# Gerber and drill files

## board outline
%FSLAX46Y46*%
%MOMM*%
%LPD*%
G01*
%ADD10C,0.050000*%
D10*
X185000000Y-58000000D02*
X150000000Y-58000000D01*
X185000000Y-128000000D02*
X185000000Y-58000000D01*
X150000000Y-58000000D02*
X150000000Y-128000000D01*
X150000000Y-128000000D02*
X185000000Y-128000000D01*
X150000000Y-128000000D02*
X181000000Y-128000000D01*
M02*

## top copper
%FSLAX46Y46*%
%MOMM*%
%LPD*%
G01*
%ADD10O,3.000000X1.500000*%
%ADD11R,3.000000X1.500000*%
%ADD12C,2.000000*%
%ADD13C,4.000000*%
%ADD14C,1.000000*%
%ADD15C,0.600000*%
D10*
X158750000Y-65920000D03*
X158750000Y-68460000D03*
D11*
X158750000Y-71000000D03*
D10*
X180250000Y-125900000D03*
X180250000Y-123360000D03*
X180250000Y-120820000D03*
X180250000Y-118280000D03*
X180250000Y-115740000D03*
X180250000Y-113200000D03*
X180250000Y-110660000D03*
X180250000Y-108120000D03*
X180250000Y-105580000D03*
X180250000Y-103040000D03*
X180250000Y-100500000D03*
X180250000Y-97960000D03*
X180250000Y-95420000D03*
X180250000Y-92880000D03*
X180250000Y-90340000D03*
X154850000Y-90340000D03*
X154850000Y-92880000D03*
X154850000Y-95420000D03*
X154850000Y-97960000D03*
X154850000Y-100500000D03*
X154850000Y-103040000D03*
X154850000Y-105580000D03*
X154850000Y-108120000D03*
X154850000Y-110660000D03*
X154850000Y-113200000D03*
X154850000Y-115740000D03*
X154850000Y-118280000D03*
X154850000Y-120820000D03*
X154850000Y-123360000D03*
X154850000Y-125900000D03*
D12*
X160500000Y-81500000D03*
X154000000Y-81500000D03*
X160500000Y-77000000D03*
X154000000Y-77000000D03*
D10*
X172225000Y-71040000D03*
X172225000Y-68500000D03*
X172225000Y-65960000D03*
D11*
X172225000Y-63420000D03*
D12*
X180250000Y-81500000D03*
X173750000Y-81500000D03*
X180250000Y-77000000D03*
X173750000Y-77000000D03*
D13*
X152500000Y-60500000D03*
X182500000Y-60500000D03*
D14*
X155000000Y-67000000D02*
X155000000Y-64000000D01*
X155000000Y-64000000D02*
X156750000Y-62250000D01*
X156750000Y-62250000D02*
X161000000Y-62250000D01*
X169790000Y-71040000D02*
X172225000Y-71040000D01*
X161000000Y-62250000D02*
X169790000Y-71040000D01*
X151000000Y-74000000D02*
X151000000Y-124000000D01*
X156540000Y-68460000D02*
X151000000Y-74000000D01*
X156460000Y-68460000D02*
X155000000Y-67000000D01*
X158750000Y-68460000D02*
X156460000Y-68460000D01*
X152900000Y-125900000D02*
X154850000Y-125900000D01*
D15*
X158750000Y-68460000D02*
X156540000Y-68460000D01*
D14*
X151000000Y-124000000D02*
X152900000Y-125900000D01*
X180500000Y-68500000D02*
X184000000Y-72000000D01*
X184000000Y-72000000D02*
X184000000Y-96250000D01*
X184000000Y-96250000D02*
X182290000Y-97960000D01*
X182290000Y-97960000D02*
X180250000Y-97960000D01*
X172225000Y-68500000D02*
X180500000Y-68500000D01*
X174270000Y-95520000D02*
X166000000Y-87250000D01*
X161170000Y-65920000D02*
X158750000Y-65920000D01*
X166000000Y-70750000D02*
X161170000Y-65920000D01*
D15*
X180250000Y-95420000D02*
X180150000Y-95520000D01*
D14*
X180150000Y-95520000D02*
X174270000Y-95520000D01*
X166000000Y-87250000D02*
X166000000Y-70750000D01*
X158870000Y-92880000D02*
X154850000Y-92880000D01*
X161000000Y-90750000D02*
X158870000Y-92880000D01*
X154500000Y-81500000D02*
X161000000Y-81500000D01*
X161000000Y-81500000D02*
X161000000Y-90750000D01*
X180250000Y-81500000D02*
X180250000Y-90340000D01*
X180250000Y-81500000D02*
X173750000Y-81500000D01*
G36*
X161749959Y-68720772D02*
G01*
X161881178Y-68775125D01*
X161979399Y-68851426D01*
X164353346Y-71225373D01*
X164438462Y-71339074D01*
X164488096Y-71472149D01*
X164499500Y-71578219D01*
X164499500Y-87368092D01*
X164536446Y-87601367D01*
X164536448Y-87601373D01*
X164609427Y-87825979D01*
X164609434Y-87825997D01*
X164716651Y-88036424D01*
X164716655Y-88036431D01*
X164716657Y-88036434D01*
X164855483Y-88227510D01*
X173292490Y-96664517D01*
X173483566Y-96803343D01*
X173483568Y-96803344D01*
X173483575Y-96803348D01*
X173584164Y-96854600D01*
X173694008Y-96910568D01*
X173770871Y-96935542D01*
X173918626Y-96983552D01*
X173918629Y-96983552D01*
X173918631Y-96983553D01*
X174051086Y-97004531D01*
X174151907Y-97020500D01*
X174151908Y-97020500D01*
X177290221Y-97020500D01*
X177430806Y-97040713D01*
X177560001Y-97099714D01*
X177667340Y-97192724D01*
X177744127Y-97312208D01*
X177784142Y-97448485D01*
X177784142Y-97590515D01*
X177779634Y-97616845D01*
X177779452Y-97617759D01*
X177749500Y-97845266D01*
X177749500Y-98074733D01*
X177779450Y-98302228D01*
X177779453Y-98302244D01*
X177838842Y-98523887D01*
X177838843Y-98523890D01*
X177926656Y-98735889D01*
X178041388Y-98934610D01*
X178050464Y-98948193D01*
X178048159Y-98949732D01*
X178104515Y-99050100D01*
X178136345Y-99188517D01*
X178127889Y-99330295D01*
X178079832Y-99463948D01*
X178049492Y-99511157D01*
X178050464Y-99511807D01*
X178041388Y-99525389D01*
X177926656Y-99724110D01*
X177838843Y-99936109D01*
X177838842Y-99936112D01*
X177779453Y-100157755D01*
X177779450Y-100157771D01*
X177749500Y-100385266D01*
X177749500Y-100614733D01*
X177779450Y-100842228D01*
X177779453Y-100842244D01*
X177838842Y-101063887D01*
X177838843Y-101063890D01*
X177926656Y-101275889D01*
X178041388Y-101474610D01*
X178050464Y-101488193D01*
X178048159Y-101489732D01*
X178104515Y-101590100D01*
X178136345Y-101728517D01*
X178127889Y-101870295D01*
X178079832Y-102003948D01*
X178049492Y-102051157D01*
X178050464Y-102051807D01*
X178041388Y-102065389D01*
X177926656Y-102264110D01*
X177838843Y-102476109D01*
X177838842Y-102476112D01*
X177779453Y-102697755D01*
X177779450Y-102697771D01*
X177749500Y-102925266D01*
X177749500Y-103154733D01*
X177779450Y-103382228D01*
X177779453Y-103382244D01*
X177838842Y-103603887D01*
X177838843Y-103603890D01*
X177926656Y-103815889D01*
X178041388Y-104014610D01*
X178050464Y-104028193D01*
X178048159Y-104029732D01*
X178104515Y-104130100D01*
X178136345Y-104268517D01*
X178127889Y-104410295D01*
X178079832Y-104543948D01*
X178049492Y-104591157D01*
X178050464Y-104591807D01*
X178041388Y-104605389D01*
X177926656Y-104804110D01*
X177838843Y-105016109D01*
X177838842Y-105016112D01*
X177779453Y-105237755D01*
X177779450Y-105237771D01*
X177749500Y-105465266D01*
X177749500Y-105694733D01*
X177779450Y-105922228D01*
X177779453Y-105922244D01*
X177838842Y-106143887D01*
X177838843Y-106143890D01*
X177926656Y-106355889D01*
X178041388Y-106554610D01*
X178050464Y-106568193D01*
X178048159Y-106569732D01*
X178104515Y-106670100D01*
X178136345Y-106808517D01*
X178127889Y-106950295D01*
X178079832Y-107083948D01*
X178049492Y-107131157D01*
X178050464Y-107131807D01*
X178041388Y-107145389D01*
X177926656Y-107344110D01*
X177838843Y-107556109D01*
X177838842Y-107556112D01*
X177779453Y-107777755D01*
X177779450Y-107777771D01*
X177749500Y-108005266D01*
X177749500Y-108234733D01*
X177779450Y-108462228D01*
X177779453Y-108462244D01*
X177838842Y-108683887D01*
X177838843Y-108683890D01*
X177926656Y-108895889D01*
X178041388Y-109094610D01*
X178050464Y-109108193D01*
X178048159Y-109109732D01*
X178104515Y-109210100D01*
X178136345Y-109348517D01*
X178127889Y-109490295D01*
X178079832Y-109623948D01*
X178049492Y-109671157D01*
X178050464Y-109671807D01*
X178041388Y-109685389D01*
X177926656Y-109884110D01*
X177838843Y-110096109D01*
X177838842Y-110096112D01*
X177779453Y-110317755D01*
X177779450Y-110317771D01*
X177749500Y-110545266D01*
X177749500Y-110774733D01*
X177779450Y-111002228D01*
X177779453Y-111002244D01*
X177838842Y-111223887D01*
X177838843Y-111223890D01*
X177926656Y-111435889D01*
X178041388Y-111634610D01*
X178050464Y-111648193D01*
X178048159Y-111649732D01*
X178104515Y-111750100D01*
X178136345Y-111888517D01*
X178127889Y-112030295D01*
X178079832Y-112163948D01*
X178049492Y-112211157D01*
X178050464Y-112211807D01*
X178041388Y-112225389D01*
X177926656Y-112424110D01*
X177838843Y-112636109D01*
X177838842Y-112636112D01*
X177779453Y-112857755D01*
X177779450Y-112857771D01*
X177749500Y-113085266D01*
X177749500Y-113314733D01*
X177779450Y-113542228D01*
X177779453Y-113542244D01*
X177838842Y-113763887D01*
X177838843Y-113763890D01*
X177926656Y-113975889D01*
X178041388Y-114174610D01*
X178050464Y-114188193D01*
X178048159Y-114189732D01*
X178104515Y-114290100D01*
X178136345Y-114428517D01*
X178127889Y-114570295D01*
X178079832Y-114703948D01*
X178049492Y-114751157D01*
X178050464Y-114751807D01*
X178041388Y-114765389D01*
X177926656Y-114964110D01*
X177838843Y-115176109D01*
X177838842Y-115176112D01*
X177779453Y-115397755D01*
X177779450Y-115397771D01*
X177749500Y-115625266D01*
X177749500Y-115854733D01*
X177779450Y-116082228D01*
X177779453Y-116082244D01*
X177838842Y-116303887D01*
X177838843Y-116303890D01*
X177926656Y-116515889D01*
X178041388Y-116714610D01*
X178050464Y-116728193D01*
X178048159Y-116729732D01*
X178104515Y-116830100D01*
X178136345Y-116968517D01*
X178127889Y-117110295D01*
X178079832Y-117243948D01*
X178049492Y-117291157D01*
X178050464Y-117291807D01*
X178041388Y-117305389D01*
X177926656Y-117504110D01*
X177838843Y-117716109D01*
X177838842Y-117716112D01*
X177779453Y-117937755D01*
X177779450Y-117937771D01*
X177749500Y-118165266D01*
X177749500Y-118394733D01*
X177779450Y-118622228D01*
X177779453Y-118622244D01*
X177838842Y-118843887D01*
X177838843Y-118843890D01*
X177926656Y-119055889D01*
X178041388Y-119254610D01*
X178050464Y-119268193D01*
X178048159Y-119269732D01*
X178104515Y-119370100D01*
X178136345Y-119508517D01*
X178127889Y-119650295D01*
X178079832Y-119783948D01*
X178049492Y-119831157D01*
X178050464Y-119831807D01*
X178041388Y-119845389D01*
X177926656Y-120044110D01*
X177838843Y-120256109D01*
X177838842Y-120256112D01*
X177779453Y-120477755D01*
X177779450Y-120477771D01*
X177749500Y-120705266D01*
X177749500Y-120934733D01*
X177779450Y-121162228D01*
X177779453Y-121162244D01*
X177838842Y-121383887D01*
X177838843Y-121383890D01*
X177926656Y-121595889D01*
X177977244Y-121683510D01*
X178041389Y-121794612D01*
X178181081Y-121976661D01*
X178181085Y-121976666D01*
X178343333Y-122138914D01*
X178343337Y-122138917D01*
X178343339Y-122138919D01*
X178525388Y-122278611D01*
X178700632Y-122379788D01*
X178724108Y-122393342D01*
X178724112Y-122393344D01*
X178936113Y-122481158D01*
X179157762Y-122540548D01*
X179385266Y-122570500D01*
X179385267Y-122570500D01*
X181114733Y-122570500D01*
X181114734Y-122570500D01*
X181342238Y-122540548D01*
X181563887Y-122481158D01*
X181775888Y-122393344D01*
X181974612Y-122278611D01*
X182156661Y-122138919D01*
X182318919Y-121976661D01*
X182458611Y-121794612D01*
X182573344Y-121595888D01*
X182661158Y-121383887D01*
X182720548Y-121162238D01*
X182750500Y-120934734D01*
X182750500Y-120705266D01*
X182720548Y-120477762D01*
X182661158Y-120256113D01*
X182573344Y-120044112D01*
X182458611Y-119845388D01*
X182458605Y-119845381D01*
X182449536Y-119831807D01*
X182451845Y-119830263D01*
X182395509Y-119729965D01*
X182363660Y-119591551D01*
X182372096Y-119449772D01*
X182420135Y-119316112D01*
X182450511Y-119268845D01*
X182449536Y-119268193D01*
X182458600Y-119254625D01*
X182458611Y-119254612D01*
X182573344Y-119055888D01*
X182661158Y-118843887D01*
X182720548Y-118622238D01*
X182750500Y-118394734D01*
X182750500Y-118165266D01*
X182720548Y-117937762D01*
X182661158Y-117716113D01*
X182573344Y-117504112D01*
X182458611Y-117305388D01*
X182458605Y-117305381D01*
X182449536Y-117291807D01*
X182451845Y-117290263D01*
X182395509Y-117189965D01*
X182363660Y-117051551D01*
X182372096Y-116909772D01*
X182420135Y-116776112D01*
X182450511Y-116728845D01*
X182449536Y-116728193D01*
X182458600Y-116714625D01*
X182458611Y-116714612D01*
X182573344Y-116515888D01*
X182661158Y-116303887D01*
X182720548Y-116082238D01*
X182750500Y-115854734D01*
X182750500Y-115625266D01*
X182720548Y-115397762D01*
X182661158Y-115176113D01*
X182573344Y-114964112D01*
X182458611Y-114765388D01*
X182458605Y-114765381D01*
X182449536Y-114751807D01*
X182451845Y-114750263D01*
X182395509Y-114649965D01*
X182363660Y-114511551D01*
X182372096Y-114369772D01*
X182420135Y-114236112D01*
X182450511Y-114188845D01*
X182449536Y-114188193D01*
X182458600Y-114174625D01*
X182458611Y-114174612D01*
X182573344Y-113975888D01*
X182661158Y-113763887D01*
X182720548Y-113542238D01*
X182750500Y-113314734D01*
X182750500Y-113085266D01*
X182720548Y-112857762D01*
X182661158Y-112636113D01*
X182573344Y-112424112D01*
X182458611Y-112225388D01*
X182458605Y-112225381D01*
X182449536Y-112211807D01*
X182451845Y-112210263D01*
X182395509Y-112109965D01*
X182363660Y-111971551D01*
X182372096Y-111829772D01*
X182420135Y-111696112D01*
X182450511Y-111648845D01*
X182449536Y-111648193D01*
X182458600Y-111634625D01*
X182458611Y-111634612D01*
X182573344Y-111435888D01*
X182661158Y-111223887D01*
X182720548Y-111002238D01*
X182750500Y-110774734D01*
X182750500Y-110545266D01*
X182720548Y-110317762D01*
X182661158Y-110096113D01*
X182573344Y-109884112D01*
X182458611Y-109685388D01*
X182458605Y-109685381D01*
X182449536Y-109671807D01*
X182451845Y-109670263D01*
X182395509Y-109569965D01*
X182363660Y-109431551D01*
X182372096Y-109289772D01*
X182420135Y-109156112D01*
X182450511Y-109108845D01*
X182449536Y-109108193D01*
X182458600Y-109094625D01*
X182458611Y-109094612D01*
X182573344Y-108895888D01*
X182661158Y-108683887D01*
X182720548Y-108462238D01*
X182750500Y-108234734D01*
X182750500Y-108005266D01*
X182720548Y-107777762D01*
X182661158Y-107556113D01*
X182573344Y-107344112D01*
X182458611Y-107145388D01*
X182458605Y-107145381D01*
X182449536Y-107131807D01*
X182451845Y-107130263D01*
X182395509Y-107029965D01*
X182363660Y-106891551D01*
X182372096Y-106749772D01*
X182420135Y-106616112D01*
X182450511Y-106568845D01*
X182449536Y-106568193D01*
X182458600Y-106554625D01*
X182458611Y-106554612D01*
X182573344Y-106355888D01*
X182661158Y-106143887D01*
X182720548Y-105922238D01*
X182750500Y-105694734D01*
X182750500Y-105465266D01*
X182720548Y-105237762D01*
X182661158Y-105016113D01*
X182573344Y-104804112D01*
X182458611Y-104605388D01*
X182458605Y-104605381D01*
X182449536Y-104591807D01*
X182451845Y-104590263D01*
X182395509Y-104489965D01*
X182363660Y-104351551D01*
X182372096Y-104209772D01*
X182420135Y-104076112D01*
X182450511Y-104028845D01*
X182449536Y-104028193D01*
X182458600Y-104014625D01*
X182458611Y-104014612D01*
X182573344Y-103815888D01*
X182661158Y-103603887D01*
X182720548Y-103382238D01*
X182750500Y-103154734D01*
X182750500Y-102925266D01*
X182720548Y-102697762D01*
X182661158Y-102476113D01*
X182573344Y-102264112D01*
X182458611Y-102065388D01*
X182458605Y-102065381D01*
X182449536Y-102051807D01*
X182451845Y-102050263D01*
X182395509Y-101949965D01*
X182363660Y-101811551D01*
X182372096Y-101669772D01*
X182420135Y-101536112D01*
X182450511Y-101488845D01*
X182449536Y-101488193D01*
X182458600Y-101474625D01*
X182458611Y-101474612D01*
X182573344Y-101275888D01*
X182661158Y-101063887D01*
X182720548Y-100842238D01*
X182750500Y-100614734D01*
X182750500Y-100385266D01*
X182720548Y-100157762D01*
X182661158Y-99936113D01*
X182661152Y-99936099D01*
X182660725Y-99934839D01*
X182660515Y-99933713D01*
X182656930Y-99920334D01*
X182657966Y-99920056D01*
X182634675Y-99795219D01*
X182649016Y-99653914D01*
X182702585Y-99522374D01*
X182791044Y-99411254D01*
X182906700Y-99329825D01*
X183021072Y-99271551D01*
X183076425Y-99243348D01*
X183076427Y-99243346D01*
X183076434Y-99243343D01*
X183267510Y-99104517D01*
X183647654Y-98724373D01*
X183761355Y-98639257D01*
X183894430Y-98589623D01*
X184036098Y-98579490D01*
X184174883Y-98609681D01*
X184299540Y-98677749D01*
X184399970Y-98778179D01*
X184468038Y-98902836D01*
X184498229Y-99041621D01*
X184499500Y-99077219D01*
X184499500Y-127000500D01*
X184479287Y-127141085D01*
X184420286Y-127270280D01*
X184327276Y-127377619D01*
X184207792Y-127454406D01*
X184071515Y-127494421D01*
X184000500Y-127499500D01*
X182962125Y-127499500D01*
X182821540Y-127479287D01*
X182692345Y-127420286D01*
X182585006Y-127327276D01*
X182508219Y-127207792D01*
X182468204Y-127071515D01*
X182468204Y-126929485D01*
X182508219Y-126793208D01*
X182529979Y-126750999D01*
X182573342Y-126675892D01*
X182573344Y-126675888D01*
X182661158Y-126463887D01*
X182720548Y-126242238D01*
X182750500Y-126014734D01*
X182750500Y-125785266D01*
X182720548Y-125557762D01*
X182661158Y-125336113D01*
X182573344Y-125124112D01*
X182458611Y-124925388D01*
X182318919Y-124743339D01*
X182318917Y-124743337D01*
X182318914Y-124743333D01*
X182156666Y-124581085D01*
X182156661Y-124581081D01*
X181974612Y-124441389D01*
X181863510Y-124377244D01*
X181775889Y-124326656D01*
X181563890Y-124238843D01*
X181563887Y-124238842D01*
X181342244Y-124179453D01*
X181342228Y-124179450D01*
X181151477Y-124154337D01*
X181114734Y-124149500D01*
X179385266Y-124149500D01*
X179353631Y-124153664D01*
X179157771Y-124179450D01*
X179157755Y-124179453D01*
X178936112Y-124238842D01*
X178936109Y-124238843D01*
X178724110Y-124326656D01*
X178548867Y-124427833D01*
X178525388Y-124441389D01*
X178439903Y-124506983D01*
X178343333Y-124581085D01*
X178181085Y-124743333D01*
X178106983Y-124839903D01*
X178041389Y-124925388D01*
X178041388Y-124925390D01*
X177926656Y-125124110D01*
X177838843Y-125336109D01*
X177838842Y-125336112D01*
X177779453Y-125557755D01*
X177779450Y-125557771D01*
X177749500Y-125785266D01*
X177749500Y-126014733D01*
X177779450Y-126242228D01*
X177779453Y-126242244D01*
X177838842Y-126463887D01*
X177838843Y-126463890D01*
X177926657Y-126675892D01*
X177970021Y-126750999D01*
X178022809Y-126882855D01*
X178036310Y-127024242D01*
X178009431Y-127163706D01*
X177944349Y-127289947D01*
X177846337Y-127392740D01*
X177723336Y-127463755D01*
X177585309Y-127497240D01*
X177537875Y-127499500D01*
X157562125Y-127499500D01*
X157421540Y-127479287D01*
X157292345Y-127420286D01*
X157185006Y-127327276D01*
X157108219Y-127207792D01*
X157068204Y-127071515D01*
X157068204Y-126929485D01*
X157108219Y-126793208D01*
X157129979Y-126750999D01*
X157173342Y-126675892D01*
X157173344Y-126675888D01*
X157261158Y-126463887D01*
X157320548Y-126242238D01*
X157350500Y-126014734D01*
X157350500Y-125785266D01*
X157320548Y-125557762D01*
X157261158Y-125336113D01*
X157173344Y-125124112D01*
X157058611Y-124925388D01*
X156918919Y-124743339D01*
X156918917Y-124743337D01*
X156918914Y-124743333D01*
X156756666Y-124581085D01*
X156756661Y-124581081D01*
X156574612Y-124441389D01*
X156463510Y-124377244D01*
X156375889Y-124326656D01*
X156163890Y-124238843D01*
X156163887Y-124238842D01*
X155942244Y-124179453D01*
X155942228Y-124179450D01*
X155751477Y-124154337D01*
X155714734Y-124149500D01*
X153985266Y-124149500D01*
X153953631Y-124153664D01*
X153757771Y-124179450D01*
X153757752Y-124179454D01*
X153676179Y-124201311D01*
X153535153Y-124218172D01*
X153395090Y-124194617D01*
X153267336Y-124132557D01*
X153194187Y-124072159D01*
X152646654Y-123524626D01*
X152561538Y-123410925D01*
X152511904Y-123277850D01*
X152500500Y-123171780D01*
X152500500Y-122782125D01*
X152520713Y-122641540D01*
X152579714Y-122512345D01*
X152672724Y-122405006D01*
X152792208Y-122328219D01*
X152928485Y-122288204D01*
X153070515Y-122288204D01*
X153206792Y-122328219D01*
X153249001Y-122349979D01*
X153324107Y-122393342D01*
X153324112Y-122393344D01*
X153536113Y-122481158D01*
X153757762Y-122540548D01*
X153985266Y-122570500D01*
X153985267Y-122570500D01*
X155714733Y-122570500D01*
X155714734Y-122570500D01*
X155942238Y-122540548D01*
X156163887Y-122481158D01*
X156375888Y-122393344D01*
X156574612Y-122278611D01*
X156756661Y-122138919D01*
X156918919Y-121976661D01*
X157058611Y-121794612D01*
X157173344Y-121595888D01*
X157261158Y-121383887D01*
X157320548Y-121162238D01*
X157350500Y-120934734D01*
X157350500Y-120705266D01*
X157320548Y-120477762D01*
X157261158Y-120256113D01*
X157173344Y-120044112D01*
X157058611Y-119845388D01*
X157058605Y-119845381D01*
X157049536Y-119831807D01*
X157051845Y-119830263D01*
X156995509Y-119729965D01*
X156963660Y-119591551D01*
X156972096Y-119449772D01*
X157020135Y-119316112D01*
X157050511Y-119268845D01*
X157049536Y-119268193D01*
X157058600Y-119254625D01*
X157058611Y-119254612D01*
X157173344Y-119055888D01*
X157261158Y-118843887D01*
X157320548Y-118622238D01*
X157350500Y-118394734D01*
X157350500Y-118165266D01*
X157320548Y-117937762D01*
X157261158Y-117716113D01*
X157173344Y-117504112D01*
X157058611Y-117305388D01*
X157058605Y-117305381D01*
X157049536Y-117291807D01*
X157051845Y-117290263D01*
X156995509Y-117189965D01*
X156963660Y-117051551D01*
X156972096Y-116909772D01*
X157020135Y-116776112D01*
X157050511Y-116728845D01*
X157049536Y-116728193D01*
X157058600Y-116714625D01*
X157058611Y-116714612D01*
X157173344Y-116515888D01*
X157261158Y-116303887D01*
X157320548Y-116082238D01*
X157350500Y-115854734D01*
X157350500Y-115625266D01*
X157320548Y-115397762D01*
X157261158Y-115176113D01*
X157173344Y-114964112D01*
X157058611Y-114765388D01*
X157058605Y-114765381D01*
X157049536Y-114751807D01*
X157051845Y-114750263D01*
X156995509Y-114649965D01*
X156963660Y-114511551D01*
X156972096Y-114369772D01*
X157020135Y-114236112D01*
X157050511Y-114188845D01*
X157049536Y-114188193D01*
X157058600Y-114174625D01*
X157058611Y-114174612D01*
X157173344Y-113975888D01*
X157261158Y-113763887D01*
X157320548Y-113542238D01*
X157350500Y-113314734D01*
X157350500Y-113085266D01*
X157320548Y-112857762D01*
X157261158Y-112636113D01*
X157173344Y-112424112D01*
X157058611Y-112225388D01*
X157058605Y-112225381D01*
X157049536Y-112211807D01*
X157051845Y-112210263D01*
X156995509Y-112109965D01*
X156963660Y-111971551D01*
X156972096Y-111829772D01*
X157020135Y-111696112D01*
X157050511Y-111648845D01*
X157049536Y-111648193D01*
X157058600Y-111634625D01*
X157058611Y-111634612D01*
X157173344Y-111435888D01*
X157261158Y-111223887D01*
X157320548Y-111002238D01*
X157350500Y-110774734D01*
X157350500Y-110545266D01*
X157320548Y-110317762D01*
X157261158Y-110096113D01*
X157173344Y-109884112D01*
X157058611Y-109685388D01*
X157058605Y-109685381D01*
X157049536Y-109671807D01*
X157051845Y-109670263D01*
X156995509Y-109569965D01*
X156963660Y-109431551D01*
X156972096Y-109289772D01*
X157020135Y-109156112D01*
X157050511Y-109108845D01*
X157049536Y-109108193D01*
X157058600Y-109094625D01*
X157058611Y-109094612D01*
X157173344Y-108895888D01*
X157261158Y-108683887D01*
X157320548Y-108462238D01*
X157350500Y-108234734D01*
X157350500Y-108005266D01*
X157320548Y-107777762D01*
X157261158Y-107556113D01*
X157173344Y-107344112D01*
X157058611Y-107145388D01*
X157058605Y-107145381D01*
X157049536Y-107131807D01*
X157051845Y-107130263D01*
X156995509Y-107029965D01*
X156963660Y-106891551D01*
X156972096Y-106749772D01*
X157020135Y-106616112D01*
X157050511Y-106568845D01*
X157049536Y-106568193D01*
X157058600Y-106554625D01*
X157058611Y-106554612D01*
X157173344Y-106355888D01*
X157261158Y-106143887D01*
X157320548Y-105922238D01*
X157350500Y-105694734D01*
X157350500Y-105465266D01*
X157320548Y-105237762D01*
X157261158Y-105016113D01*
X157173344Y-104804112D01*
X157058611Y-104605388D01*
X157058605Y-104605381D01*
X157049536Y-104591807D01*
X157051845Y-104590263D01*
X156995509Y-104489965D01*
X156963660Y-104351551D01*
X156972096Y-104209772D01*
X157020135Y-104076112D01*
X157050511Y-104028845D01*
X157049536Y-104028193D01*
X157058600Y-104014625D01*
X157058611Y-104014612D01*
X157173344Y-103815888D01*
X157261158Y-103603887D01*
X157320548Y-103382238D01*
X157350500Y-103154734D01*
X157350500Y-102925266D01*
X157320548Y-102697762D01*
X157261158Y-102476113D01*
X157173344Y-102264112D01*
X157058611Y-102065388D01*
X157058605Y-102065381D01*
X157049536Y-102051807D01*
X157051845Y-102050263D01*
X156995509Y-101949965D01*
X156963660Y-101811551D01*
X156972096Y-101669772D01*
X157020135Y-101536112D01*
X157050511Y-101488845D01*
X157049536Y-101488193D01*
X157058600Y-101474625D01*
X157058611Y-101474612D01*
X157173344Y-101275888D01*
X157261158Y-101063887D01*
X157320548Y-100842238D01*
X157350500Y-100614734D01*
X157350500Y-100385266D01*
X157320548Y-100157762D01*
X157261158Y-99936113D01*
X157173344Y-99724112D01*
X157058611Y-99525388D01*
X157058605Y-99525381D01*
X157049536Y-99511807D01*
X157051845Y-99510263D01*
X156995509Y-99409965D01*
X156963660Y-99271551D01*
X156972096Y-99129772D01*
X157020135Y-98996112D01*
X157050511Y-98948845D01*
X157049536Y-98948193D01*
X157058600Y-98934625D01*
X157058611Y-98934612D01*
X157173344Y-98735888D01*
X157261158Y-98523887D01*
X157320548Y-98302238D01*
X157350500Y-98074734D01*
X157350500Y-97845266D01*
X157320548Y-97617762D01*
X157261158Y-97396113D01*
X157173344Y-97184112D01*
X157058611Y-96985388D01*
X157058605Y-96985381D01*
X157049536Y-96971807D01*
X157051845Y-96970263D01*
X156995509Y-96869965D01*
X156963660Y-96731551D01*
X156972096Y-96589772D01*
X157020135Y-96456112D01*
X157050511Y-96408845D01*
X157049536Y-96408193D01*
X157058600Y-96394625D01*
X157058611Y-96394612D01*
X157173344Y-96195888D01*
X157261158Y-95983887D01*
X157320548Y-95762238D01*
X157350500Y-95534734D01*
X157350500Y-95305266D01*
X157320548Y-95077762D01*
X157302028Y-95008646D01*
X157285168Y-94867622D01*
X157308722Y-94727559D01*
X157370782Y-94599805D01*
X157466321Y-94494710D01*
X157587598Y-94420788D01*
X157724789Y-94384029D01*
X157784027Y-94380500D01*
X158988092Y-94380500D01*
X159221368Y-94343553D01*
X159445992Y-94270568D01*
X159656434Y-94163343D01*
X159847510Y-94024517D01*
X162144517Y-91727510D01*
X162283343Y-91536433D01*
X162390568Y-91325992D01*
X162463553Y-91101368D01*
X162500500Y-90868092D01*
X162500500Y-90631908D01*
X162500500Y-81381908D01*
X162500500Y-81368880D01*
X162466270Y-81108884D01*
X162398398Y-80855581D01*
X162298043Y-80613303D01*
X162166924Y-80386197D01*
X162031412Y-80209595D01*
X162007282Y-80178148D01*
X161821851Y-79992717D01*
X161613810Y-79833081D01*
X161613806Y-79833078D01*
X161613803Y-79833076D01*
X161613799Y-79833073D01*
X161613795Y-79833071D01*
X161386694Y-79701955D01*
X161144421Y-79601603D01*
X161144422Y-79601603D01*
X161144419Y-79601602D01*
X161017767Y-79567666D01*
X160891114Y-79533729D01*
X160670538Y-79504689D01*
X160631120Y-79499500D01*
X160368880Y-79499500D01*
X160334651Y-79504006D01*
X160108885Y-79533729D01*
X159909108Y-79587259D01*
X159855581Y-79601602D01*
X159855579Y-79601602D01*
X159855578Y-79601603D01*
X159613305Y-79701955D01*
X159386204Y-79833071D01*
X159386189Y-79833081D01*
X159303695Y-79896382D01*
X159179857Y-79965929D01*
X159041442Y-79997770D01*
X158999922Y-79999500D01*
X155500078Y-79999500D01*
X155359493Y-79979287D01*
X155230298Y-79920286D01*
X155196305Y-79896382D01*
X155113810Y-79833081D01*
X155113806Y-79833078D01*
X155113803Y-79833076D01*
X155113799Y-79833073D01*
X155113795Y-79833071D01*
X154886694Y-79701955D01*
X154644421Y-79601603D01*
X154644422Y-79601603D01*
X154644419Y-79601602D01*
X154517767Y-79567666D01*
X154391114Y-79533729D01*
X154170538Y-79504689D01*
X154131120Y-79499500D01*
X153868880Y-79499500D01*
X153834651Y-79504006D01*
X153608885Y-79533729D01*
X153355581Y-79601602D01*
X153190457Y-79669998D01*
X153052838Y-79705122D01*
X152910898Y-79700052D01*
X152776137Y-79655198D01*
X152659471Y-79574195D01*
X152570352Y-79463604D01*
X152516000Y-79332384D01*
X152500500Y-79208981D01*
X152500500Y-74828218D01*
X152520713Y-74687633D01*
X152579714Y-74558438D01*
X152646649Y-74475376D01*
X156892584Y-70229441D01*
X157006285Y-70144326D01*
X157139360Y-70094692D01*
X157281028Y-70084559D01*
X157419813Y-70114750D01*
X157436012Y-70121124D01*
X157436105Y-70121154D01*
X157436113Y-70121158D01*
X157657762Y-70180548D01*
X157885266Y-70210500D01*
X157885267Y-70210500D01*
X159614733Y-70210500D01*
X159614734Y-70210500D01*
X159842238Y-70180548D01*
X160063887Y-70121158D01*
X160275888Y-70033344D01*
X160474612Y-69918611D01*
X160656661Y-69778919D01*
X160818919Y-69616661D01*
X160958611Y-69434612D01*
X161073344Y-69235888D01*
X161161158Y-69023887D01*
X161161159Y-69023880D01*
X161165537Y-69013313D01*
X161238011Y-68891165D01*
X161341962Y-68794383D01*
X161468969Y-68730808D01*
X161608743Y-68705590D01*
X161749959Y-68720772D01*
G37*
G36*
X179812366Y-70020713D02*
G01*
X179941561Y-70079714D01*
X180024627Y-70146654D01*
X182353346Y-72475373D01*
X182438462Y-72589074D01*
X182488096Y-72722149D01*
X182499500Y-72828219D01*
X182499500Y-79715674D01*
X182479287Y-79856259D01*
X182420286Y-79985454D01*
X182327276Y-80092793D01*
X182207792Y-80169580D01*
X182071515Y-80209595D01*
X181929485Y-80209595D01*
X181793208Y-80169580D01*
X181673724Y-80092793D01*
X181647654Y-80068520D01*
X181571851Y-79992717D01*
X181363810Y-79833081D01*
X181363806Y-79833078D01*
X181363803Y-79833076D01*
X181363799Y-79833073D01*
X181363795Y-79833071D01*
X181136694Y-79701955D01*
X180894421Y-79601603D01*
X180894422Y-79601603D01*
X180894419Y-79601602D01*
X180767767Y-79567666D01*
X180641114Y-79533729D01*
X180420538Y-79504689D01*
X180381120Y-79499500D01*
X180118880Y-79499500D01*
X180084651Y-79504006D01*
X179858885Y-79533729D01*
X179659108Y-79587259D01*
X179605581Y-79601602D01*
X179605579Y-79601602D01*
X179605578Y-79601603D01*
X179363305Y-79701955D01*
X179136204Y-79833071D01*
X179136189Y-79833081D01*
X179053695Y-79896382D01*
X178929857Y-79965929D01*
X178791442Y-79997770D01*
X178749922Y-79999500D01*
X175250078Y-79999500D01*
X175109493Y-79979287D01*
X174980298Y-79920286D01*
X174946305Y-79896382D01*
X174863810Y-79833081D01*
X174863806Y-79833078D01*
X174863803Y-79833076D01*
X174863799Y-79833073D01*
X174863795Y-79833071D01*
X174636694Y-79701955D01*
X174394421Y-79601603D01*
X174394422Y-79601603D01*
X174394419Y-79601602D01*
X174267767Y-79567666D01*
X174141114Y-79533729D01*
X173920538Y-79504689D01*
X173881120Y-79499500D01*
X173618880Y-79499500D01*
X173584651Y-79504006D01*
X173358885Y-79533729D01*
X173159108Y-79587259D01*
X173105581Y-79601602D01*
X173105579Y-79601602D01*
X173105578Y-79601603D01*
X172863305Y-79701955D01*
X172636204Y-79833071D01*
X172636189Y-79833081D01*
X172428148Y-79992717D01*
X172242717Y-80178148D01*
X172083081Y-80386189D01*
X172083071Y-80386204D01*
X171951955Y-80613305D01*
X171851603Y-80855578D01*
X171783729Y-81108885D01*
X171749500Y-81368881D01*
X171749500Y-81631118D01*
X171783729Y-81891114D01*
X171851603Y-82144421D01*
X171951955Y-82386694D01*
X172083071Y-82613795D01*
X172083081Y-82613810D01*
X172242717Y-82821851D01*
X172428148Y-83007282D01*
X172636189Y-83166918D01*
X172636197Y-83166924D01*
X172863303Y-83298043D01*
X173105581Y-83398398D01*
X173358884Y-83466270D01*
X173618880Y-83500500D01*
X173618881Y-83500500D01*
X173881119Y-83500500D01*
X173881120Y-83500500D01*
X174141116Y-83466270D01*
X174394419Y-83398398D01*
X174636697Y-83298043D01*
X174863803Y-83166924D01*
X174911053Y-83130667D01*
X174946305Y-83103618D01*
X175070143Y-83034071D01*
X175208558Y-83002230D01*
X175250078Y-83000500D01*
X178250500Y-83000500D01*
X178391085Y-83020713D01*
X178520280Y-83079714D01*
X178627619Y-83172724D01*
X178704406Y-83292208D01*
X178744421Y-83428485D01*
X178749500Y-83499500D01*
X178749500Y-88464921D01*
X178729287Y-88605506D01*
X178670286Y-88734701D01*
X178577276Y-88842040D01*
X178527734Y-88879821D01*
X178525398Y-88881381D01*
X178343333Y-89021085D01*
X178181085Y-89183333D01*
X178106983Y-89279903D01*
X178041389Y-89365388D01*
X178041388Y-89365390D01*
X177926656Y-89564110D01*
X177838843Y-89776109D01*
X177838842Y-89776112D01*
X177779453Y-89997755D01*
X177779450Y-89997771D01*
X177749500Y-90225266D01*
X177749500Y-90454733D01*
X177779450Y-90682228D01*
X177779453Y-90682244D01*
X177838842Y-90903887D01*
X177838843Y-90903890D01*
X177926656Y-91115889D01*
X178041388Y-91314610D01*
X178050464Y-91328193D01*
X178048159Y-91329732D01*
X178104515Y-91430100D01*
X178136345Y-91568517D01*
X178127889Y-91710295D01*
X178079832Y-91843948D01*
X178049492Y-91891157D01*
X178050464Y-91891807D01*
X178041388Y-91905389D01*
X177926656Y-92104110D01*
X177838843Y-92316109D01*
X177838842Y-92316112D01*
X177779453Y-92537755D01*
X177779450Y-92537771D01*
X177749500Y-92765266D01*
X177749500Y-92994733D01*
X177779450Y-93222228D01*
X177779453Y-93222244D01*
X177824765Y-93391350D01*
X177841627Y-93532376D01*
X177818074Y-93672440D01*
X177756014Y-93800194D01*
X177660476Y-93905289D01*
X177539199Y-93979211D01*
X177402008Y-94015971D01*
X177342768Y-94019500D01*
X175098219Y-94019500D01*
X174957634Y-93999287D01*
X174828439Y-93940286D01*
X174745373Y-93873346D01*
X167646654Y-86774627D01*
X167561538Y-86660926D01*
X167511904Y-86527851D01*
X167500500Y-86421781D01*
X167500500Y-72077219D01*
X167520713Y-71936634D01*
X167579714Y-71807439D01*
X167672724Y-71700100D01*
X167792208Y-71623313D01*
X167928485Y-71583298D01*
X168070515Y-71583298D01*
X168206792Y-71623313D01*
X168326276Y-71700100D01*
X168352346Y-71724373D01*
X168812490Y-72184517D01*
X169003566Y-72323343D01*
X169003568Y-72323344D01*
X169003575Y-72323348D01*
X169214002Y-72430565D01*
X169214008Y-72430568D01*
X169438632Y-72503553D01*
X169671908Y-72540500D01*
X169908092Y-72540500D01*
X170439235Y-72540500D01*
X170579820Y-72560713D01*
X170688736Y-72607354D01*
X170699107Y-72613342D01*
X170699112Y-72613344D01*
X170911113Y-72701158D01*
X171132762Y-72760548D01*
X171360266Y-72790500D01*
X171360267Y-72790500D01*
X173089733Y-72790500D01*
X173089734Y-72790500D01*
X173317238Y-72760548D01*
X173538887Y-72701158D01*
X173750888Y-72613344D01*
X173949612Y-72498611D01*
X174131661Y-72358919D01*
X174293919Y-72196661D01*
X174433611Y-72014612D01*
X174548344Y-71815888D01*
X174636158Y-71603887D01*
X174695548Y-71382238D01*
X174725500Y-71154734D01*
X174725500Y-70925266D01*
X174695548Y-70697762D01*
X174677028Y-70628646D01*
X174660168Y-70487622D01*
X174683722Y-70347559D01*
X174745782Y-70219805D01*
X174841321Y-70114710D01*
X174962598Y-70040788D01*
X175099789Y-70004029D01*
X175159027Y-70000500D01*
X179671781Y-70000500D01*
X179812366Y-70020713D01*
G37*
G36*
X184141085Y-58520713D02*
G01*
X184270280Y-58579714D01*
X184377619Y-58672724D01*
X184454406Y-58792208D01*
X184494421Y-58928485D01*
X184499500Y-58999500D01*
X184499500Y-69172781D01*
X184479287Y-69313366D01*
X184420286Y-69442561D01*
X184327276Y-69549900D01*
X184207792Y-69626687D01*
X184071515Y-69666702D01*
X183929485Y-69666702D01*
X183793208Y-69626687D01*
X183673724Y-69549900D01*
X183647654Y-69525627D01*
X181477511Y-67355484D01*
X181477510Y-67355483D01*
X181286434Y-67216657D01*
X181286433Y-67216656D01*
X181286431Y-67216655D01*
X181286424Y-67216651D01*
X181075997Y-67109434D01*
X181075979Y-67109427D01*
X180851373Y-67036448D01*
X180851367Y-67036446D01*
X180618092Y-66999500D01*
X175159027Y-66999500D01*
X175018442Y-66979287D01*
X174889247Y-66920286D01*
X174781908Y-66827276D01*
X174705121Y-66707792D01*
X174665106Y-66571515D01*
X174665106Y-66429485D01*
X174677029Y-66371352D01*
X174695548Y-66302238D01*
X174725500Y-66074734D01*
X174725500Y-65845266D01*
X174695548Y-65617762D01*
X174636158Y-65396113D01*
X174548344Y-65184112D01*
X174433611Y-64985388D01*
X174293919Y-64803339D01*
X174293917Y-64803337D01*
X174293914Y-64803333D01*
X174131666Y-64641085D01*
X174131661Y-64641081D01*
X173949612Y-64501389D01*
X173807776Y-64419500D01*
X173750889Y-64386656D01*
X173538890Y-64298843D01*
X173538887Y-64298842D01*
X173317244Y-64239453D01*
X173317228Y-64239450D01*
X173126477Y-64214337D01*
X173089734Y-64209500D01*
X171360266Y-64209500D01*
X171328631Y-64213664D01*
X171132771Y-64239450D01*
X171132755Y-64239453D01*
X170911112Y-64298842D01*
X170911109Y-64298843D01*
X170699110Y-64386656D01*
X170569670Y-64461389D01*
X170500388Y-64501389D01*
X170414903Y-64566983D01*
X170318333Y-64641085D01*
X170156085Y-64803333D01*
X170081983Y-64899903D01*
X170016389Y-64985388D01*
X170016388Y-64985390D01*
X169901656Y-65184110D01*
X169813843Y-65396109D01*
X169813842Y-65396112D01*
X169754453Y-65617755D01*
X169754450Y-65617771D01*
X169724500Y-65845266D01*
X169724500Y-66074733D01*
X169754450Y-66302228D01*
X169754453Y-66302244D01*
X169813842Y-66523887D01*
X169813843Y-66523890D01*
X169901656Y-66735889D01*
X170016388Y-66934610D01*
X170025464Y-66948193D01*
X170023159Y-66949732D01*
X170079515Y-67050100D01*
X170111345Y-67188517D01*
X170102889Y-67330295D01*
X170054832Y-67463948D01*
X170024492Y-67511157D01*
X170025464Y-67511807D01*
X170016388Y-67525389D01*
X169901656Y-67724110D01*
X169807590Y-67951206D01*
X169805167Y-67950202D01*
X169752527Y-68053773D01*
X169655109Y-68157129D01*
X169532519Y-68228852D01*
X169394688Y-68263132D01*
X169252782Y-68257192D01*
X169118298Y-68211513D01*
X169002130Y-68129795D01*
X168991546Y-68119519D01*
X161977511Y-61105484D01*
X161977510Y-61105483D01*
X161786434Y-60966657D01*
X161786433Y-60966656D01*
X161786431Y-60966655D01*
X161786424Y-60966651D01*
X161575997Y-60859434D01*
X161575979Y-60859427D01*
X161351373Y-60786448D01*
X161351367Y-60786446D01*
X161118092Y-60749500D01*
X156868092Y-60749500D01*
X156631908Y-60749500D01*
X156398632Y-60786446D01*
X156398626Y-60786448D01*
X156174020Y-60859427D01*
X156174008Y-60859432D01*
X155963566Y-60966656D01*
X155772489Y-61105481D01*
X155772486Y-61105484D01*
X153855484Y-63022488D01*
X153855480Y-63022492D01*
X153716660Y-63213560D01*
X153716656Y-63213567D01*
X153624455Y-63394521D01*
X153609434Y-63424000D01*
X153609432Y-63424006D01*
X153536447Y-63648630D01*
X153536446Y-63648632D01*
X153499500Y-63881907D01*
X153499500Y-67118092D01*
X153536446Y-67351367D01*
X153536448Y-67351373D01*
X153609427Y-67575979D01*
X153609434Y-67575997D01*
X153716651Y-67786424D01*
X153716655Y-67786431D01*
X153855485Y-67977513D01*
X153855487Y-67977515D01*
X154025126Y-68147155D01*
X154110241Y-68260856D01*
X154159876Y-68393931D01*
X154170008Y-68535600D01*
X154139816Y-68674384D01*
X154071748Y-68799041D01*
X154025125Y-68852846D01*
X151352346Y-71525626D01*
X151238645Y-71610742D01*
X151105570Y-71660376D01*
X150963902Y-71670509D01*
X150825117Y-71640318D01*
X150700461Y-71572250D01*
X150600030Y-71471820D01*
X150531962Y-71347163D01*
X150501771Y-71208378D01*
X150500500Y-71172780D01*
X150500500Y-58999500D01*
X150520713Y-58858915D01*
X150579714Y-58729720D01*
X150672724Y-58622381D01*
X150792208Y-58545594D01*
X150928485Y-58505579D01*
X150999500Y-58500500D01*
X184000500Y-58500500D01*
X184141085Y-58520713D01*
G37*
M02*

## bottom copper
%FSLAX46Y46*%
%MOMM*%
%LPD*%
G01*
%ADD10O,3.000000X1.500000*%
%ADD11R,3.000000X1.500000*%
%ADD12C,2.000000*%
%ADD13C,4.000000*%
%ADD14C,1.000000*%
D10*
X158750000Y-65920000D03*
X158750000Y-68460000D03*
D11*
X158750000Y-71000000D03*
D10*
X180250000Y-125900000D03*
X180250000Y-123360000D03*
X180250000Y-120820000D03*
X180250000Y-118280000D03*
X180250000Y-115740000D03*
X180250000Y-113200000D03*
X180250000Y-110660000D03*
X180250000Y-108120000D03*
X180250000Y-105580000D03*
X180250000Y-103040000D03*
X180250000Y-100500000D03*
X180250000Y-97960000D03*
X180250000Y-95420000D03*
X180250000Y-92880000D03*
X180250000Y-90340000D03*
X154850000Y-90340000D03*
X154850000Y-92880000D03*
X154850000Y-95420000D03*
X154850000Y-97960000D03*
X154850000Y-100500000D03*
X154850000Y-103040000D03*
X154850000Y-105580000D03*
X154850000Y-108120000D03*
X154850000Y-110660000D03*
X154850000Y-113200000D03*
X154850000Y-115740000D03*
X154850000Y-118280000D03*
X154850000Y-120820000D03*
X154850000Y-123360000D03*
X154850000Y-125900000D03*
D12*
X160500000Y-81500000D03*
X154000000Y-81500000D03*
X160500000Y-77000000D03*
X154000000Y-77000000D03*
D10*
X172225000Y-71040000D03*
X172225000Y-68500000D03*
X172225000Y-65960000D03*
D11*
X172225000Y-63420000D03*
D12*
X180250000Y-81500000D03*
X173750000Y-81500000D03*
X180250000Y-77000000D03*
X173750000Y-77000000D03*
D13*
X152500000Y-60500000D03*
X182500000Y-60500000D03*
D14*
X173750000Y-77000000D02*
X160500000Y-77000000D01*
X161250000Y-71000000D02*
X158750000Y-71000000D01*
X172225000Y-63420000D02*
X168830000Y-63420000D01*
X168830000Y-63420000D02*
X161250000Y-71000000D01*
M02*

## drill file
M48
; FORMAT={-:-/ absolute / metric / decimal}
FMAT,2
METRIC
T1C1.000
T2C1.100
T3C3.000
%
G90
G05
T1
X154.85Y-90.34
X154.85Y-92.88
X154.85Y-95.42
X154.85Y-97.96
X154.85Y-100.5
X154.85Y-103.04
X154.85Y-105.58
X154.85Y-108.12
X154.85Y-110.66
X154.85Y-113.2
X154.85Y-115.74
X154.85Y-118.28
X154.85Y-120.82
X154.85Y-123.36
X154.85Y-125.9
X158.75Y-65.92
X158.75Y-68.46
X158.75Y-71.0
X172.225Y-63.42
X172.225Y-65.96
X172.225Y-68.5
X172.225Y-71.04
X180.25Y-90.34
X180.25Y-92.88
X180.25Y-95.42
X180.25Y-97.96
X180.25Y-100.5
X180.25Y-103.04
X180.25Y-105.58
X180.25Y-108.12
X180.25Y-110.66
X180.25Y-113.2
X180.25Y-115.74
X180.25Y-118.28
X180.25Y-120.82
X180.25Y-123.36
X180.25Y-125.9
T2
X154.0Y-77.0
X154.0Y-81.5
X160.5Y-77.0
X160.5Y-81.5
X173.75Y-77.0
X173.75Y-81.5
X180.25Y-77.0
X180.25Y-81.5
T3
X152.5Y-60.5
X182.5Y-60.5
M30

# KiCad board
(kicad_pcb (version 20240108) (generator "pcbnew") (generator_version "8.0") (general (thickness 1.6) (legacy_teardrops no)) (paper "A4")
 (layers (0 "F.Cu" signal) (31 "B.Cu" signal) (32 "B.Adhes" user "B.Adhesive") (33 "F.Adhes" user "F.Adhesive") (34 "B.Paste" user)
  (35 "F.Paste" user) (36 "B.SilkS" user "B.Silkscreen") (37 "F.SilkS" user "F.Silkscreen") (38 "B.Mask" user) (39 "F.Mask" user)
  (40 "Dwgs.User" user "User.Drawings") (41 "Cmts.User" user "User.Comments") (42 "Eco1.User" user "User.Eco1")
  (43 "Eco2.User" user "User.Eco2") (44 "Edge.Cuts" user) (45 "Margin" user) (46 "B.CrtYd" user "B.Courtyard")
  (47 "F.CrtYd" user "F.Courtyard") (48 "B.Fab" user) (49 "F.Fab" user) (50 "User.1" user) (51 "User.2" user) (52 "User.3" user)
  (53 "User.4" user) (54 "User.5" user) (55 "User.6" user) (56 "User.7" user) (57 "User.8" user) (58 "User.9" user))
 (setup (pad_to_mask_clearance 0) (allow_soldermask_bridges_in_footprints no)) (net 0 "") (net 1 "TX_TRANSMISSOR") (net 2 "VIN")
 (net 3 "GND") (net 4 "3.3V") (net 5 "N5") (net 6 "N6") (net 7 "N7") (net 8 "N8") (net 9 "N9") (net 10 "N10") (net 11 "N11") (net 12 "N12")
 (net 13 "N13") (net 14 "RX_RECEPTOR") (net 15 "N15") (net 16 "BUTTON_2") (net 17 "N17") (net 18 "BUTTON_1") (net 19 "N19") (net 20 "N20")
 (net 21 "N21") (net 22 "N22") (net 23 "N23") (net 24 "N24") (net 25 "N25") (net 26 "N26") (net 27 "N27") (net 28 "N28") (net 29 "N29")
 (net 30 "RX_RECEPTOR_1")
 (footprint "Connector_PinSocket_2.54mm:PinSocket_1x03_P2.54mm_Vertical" (layer "F.Cu") (at 158.75 65.92)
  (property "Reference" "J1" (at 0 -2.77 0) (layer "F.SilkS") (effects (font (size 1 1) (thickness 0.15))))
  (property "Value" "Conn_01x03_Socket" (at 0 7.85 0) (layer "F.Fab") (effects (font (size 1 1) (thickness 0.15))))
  (pad "1" thru_hole oval (at 0 0) (size 3 1.5) (drill 1) (layers "*.Cu" "*.Mask") (remove_unused_layers no) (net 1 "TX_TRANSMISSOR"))
  (pad "2" thru_hole oval (at 0 2.54) (size 3 1.5) (drill 1) (layers "*.Cu" "*.Mask") (remove_unused_layers no) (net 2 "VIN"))
  (pad "3" thru_hole rect (at 0 5.08) (size 3 1.5) (drill 1) (layers "*.Cu" "*.Mask") (remove_unused_layers no) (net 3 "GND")))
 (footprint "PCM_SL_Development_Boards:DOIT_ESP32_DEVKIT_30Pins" (layer "F.Cu") (at 180.25 125.9 180)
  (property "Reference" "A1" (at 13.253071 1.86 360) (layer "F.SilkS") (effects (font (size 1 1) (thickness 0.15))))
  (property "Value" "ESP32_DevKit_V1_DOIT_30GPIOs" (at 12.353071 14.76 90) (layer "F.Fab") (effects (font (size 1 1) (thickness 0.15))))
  (pad "1" thru_hole oval (at 0 0 90) (size 1.5 3) (drill 1) (layers "*.Cu" "*.Mask") (remove_unused_layers no) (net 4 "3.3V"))
  (pad "2" thru_hole oval (at 0 2.54 90) (size 1.5 3) (drill 1) (layers "*.Cu" "*.Mask") (remove_unused_layers no) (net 3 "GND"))
  (pad "3" thru_hole oval (at 0 5.08 90) (size 1.5 3) (drill 1) (layers "*.Cu" "*.Mask") (remove_unused_layers no) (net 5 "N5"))
  (pad "4" thru_hole oval (at 0 7.62 90) (size 1.5 3) (drill 1) (layers "*.Cu" "*.Mask") (remove_unused_layers no) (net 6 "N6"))
  (pad "5" thru_hole oval (at 0 10.16 90) (size 1.5 3) (drill 1) (layers "*.Cu" "*.Mask") (remove_unused_layers no) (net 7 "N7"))
  (pad "6" thru_hole oval (at 0 12.7 90) (size 1.5 3) (drill 1) (layers "*.Cu" "*.Mask") (remove_unused_layers no) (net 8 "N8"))
  (pad "7" thru_hole oval (at 0 15.24 90) (size 1.5 3) (drill 1) (layers "*.Cu" "*.Mask") (remove_unused_layers no) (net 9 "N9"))
  (pad "8" thru_hole oval (at 0 17.78 90) (size 1.5 3) (drill 1) (layers "*.Cu" "*.Mask") (remove_unused_layers no) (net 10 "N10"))
  (pad "9" thru_hole oval (at 0 20.32 90) (size 1.5 3) (drill 1) (layers "*.Cu" "*.Mask") (remove_unused_layers no) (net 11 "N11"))
  (pad "10" thru_hole oval (at 0 22.86 90) (size 1.5 3) (drill 1) (layers "*.Cu" "*.Mask") (remove_unused_layers no) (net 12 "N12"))
  (pad "11" thru_hole oval (at 0 25.4 90) (size 1.5 3) (drill 1) (layers "*.Cu" "*.Mask") (remove_unused_layers no) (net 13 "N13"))
  (pad "12" thru_hole oval (at 0 27.94 90) (size 1.5 3) (drill 1) (layers "*.Cu" "*.Mask") (remove_unused_layers no) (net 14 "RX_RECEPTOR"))
  (pad "13" thru_hole oval (at 0 30.48 90) (size 1.5 3) (drill 1) (layers "*.Cu" "*.Mask") (remove_unused_layers no)
   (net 1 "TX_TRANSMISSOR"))
  (pad "14" thru_hole oval (at 0 33.02 90) (size 1.5 3) (drill 1) (layers "*.Cu" "*.Mask") (remove_unused_layers no) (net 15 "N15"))
  (pad "15" thru_hole oval (at 0 35.56 90) (size 1.5 3) (drill 1) (layers "*.Cu" "*.Mask") (remove_unused_layers no) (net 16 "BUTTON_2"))
  (pad "16" thru_hole oval (at 25.4 35.56 90) (size 1.5 3) (drill 1) (layers "*.Cu" "*.Mask") (remove_unused_layers no) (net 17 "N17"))
  (pad "17" thru_hole oval (at 25.4 33.02 90) (size 1.5 3) (drill 1) (layers "*.Cu" "*.Mask") (remove_unused_layers no) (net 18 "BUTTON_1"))
  (pad "18" thru_hole oval (at 25.4 30.48 90) (size 1.5 3) (drill 1) (layers "*.Cu" "*.Mask") (remove_unused_layers no) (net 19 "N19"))
  (pad "19" thru_hole oval (at 25.4 27.94 90) (size 1.5 3) (drill 1) (layers "*.Cu" "*.Mask") (remove_unused_layers no) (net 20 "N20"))
  (pad "20" thru_hole oval (at 25.4 25.4 90) (size 1.5 3) (drill 1) (layers "*.Cu" "*.Mask") (remove_unused_layers no) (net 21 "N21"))
  (pad "21" thru_hole oval (at 25.4 22.86 90) (size 1.5 3) (drill 1) (layers "*.Cu" "*.Mask") (remove_unused_layers no) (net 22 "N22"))
  (pad "22" thru_hole oval (at 25.4 20.32 90) (size 1.5 3) (drill 1) (layers "*.Cu" "*.Mask") (remove_unused_layers no) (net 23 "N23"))
  (pad "23" thru_hole oval (at 25.4 17.78 90) (size 1.5 3) (drill 1) (layers "*.Cu" "*.Mask") (remove_unused_layers no) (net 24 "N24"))
  (pad "24" thru_hole oval (at 25.4 15.24 90) (size 1.5 3) (drill 1) (layers "*.Cu" "*.Mask") (remove_unused_layers no) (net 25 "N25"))
  (pad "25" thru_hole oval (at 25.4 12.7 90) (size 1.5 3) (drill 1) (layers "*.Cu" "*.Mask") (remove_unused_layers no) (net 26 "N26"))
  (pad "26" thru_hole oval (at 25.4 10.16 90) (size 1.5 3) (drill 1) (layers "*.Cu" "*.Mask") (remove_unused_layers no) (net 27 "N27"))
  (pad "27" thru_hole oval (at 25.4 7.62 90) (size 1.5 3) (drill 1) (layers "*.Cu" "*.Mask") (remove_unused_layers no) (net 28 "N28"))
  (pad "28" thru_hole oval (at 25.4 5.08 90) (size 1.5 3) (drill 1) (layers "*.Cu" "*.Mask") (remove_unused_layers no) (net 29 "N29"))
  (pad "29" thru_hole oval (at 25.4 2.54 90) (size 1.5 3) (drill 1) (layers "*.Cu" "*.Mask") (remove_unused_layers no) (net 3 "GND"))
  (pad "30" thru_hole oval (at 25.4 0 90) (size 1.5 3) (drill 1) (layers "*.Cu" "*.Mask") (remove_unused_layers no) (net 2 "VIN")))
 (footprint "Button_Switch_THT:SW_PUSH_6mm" (layer "F.Cu") (at 160.5 81.5 180)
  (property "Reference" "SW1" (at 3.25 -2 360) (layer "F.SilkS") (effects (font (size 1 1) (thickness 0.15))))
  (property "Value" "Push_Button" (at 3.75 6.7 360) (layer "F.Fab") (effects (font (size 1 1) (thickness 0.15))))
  (pad "1" thru_hole circle (at 0 0 270) (size 2 2) (drill 1.1) (layers "*.Cu" "*.Mask") (remove_unused_layers no) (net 18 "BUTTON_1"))
  (pad "1" thru_hole circle (at 6.5 0 270) (size 2 2) (drill 1.1) (layers "*.Cu" "*.Mask") (remove_unused_layers no) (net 18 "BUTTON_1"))
  (pad "2" thru_hole circle (at 0 4.5 270) (size 2 2) (drill 1.1) (layers "*.Cu" "*.Mask") (remove_unused_layers no) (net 3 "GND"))
  (pad "2" thru_hole circle (at 6.5 4.5 270) (size 2 2) (drill 1.1) (layers "*.Cu" "*.Mask") (remove_unused_layers no) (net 3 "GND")))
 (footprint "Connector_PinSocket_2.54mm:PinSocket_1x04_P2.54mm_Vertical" (layer "F.Cu") (at 172.225 71.04 180)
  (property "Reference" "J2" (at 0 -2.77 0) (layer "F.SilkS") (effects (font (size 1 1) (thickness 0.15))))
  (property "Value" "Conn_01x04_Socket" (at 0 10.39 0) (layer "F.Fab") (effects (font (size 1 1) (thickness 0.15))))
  (pad "1" thru_hole oval (at 0 0 180) (size 3 1.5) (drill 1) (layers "*.Cu" "*.Mask") (remove_unused_layers no) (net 2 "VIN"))
  (pad "2" thru_hole oval (at 0 2.54 180) (size 3 1.5) (drill 1) (layers "*.Cu" "*.Mask") (remove_unused_layers no) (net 14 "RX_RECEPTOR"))
  (pad "3" thru_hole oval (at 0 5.08 180) (size 3 1.5) (drill 1) (layers "*.Cu" "*.Mask") (remove_unused_layers no) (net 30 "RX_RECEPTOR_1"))
  (pad "4" thru_hole rect (at 0 7.62 180) (size 3 1.5) (drill 1) (layers "*.Cu" "*.Mask") (remove_unused_layers no) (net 3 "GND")))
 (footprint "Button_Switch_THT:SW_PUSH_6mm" (layer "F.Cu") (at 180.25 81.5 180)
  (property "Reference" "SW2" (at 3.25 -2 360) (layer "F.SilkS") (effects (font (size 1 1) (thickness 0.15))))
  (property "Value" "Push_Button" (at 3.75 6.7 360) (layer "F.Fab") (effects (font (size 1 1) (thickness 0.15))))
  (pad "1" thru_hole circle (at 0 0 270) (size 2 2) (drill 1.1) (layers "*.Cu" "*.Mask") (remove_unused_layers no) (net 16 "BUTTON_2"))
  (pad "1" thru_hole circle (at 6.5 0 270) (size 2 2) (drill 1.1) (layers "*.Cu" "*.Mask") (remove_unused_layers no) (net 16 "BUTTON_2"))
  (pad "2" thru_hole circle (at 0 4.5 270) (size 2 2) (drill 1.1) (layers "*.Cu" "*.Mask") (remove_unused_layers no) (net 3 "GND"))
  (pad "2" thru_hole circle (at 6.5 4.5 270) (size 2 2) (drill 1.1) (layers "*.Cu" "*.Mask") (remove_unused_layers no) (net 3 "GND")))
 (gr_line (start 185 58) (end 150 58) (stroke (width 0.05) (type default)) (layer "Edge.Cuts"))
 (gr_line (start 185 128) (end 185 58) (stroke (width 0.05) (type default)) (layer "Edge.Cuts"))
 (gr_line (start 150 58) (end 150 128) (stroke (width 0.05) (type default)) (layer "Edge.Cuts"))
 (gr_line (start 150 128) (end 185 128) (stroke (width 0.05) (type default)) (layer "Edge.Cuts"))
 (gr_line (start 150 128) (end 181 128) (stroke (width 0.05) (type default)) (layer "Edge.Cuts"))
 (segment (start 155 67) (end 155 64) (width 1) (layer "F.Cu") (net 2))
 (segment (start 155 64) (end 156.75 62.25) (width 1) (layer "F.Cu") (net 2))
 (segment (start 156.75 62.25) (end 161 62.25) (width 1) (layer "F.Cu") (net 2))
 (segment (start 169.79 71.04) (end 172.225 71.04) (width 1) (layer "F.Cu") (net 2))
 (segment (start 161 62.25) (end 169.79 71.04) (width 1) (layer "F.Cu") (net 2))
 (segment (start 151 74) (end 151 124) (width 1) (layer "F.Cu") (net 2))
 (segment (start 156.54 68.46) (end 151 74) (width 1) (layer "F.Cu") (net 2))
 (segment (start 156.46 68.46) (end 155 67) (width 1) (layer "F.Cu") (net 2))
 (segment (start 158.75 68.46) (end 156.46 68.46) (width 1) (layer "F.Cu") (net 2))
 (segment (start 152.9 125.9) (end 154.85 125.9) (width 1) (layer "F.Cu") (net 2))
 (segment (start 158.75 68.46) (end 156.54 68.46) (width 0.6) (layer "F.Cu") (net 2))
 (segment (start 151 124) (end 152.9 125.9) (width 1) (layer "F.Cu") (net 2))
 (segment (start 180.5 68.5) (end 184 72) (width 1) (layer "F.Cu") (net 14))
 (segment (start 184 72) (end 184 96.25) (width 1) (layer "F.Cu") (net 14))
 (segment (start 184 96.25) (end 182.29 97.96) (width 1) (layer "F.Cu") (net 14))
 (segment (start 182.29 97.96) (end 180.25 97.96) (width 1) (layer "F.Cu") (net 14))
 (segment (start 172.225 68.5) (end 180.5 68.5) (width 1) (layer "F.Cu") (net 14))
 (segment (start 174.27 95.52) (end 166 87.25) (width 1) (layer "F.Cu") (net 1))
 (segment (start 161.17 65.92) (end 158.75 65.92) (width 1) (layer "F.Cu") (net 1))
 (segment (start 166 70.75) (end 161.17 65.92) (width 1) (layer "F.Cu") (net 1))
 (segment (start 180.25 95.42) (end 180.15 95.52) (width 0.6) (layer "F.Cu") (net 1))
 (segment (start 180.15 95.52) (end 174.27 95.52) (width 1) (layer "F.Cu") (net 1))
 (segment (start 166 87.25) (end 166 70.75) (width 1) (layer "F.Cu") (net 1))
 (via (at 152.5 60.5) (size 4) (drill 3) (layers "F.Cu" "B.Cu") (free yes) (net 3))
 (via (at 182.5 60.5) (size 4) (drill 3) (layers "F.Cu" "B.Cu") (free yes) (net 3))
 (segment (start 173.75 77) (end 160.5 77) (width 1) (layer "B.Cu") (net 3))
 (segment (start 161.25 71) (end 158.75 71) (width 1) (layer "B.Cu") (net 3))
 (segment (start 172.225 63.42) (end 168.83 63.42) (width 1) (layer "B.Cu") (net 3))
 (segment (start 168.83 63.42) (end 161.25 71) (width 1) (layer "B.Cu") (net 3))
 (segment (start 158.87 92.88) (end 154.85 92.88) (width 1) (layer "F.Cu") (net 18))
 (segment (start 161 90.75) (end 158.87 92.88) (width 1) (layer "F.Cu") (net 18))
 (segment (start 154.5 81.5) (end 161 81.5) (width 1) (layer "F.Cu") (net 18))
 (segment (start 161 81.5) (end 161 90.75) (width 1) (layer "F.Cu") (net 18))
 (segment (start 180.25 81.5) (end 180.25 90.34) (width 1) (layer "F.Cu") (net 16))
 (segment (start 180.25 81.5) (end 173.75 81.5) (width 1) (layer "F.Cu") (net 16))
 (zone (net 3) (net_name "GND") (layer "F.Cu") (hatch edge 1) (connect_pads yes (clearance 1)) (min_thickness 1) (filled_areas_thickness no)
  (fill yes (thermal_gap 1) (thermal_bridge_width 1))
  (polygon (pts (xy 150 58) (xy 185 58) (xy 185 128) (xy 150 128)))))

